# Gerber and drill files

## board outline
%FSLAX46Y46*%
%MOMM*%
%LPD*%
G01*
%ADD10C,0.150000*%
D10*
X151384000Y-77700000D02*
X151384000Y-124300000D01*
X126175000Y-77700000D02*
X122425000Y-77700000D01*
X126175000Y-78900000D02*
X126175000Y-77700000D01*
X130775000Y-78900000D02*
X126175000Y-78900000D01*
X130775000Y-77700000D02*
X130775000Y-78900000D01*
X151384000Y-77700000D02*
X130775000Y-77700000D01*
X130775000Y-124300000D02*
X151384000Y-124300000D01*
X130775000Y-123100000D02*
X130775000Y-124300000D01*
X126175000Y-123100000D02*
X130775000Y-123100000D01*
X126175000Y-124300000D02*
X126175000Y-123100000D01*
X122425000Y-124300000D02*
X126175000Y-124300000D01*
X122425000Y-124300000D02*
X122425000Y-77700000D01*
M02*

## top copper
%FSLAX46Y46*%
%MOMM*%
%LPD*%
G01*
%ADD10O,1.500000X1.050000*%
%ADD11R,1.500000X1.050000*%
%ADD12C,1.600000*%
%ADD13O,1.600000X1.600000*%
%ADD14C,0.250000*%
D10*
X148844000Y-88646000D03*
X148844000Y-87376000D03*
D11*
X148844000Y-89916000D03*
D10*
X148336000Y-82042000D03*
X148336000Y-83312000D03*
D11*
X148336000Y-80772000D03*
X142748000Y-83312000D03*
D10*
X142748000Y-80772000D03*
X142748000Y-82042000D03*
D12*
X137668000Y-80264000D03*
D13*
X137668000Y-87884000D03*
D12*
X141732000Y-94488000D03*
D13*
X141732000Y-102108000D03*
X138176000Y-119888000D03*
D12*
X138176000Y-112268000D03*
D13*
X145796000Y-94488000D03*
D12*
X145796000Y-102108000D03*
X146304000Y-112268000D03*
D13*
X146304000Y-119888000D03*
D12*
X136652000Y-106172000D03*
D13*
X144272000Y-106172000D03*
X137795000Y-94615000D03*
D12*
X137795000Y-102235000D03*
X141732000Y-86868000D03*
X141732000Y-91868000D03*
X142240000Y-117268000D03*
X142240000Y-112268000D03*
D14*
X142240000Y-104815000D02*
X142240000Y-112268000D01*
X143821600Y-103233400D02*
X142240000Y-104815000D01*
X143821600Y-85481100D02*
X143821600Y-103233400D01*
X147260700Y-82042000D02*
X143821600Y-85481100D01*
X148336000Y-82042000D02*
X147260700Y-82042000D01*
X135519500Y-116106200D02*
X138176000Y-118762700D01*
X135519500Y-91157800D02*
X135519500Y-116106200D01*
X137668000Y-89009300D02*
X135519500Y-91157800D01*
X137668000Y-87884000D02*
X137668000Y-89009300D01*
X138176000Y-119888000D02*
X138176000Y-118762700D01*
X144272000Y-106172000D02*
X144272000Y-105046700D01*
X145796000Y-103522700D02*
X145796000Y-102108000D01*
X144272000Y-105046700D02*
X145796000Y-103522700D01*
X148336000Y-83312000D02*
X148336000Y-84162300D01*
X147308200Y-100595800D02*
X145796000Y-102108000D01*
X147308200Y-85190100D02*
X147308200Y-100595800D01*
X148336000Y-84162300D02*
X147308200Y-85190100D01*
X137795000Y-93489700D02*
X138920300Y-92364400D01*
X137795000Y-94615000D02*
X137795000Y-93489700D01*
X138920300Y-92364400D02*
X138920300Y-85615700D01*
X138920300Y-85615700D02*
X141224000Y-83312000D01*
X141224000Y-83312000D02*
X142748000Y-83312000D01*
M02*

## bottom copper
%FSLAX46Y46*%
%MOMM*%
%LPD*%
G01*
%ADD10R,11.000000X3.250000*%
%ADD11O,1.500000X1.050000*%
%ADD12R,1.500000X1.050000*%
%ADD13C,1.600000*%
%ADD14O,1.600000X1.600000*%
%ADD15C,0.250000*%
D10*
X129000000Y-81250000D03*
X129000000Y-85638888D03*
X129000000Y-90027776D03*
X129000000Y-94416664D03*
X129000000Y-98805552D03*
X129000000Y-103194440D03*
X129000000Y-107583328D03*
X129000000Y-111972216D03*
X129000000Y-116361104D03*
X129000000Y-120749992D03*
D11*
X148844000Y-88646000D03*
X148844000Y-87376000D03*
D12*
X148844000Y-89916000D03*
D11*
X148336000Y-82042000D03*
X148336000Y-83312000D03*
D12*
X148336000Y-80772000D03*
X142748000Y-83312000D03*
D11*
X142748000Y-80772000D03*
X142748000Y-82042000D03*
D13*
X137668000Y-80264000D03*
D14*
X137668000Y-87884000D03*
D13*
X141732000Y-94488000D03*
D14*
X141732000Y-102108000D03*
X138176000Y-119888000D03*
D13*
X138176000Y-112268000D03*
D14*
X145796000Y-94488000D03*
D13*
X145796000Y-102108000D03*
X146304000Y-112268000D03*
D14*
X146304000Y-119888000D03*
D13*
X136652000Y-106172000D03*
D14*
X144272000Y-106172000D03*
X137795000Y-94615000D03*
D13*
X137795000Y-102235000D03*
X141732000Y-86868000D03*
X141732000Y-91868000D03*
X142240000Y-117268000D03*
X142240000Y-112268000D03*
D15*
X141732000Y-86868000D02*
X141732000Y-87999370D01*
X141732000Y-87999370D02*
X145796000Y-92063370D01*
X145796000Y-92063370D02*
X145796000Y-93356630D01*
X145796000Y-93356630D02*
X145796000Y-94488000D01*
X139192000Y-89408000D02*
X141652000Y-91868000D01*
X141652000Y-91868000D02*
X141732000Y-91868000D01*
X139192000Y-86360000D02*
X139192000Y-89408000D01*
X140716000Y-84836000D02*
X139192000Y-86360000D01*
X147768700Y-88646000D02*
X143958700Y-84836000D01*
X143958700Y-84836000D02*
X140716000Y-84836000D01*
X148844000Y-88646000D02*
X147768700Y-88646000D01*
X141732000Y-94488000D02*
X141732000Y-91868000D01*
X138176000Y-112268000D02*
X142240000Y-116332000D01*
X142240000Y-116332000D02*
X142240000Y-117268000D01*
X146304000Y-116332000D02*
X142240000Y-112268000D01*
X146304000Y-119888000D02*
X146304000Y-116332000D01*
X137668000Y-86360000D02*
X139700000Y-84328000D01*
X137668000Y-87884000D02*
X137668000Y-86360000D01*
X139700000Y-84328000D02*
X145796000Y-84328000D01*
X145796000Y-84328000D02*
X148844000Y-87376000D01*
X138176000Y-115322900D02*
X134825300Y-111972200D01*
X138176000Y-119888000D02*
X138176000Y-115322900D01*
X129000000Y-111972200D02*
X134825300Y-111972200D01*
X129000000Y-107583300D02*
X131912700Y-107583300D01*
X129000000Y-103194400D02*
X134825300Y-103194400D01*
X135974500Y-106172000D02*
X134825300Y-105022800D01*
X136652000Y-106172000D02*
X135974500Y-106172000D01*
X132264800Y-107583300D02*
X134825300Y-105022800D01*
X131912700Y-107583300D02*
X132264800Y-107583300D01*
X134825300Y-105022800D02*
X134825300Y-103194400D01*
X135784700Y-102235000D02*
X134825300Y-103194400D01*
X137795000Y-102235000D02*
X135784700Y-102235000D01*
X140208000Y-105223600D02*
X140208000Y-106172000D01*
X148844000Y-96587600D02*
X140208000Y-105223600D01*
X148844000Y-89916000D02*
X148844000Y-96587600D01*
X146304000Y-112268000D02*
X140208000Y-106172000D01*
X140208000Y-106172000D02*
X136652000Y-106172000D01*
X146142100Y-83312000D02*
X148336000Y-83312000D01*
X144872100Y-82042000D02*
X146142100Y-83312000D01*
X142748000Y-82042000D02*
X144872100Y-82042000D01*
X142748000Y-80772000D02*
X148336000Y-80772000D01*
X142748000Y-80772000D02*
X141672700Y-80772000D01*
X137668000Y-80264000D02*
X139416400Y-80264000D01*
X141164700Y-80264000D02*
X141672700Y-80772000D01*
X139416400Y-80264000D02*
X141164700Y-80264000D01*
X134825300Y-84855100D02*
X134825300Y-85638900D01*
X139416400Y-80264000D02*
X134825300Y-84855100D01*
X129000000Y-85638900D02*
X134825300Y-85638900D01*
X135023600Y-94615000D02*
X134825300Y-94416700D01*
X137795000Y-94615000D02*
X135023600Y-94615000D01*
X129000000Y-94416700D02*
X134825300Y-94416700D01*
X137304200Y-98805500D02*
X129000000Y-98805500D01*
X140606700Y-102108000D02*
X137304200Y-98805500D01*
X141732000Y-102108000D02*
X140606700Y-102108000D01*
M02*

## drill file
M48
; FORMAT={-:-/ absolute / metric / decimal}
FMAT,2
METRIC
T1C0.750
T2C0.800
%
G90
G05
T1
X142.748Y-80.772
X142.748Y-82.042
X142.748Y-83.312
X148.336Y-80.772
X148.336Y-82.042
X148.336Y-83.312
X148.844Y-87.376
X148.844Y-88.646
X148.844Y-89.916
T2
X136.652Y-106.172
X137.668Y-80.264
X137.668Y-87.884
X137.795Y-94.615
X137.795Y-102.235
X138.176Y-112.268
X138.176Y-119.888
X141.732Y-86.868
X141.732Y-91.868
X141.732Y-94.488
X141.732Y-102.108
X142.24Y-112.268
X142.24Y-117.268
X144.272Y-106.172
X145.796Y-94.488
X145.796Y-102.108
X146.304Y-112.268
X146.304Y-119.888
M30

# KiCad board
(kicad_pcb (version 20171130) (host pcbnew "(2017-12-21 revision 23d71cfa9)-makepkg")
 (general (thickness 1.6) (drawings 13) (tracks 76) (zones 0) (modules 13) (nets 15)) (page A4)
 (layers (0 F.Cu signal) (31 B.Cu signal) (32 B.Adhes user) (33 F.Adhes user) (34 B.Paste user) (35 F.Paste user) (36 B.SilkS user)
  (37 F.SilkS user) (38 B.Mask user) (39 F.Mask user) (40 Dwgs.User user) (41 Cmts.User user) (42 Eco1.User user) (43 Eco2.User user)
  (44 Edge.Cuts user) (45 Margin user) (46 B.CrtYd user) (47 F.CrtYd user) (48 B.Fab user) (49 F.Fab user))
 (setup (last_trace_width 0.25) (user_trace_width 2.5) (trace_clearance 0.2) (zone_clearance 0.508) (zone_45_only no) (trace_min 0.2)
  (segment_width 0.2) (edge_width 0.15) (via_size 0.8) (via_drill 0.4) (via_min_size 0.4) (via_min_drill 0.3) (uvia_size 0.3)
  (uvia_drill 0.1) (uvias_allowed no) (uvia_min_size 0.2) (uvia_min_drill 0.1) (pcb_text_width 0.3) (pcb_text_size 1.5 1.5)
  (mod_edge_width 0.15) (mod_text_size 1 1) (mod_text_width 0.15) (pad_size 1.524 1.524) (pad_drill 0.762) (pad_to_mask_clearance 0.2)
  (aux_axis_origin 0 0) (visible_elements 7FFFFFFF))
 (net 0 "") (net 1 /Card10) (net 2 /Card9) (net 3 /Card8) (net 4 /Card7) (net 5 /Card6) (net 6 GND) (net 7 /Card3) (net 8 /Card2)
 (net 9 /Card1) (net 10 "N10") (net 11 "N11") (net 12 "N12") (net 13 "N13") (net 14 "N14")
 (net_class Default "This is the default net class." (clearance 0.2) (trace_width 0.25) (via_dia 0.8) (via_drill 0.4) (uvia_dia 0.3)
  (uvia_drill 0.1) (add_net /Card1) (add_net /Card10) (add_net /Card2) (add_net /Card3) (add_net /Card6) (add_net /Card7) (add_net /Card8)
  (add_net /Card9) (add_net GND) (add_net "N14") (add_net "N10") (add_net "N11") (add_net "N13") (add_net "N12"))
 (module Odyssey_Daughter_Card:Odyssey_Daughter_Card (layer F.Cu) (at 129 101)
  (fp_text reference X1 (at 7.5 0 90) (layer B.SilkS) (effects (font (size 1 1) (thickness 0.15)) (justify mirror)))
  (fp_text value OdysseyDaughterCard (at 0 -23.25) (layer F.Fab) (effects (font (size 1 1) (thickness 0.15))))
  (pad 10 smd rect (at 0 -19.75) (size 11 3.25) (layers B.Cu B.Mask) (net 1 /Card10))
  (pad 9 smd rect (at 0 -15.361112) (size 11 3.25) (layers B.Cu B.Mask) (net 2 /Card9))
  (pad 8 smd rect (at 0 -10.972224) (size 11 3.25) (layers B.Cu B.Mask) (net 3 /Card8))
  (pad 7 smd rect (at 0 -6.583336) (size 11 3.25) (layers B.Cu B.Mask) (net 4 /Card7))
  (pad 6 smd rect (at 0 -2.194448) (size 11 3.25) (layers B.Cu B.Mask) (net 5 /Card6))
  (pad 5 smd rect (at 0 2.19444) (size 11 3.25) (layers B.Cu B.Mask) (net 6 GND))
  (pad 4 smd rect (at 0 6.583328) (size 11 3.25) (layers B.Cu B.Mask) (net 6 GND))
  (pad 3 smd rect (at 0 10.972216) (size 11 3.25) (layers B.Cu B.Mask) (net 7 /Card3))
  (pad 2 smd rect (at 0 15.361104) (size 11 3.25) (layers B.Cu B.Mask) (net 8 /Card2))
  (pad 1 smd rect (at 0 19.749992) (size 11 3.25) (layers B.Cu B.Mask) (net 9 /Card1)))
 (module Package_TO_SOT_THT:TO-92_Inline (layer F.Cu) (at 148.844 89.916 90)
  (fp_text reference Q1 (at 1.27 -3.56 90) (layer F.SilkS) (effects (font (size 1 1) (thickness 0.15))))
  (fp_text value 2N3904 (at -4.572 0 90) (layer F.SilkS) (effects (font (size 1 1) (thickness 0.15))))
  (pad 2 thru_hole oval (at 1.27 0 90) (size 1.05 1.5) (drill 0.75) (layers *.Cu *.Mask) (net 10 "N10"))
  (pad 3 thru_hole oval (at 2.54 0 90) (size 1.05 1.5) (drill 0.75) (layers *.Cu *.Mask) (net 7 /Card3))
  (pad 1 thru_hole rect (at 0 0 90) (size 1.05 1.5) (drill 0.75) (layers *.Cu *.Mask) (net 6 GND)))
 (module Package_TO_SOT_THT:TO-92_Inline (layer F.Cu) (at 148.336 80.772 270)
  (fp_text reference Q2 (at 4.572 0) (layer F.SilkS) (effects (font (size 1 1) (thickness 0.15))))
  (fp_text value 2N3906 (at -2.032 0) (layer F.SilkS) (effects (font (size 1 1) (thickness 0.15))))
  (pad 2 thru_hole oval (at 1.27 0 270) (size 1.05 1.5) (drill 0.75) (layers *.Cu *.Mask) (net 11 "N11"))
  (pad 3 thru_hole oval (at 2.54 0 270) (size 1.05 1.5) (drill 0.75) (layers *.Cu *.Mask) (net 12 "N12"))
  (pad 1 thru_hole rect (at 0 0 270) (size 1.05 1.5) (drill 0.75) (layers *.Cu *.Mask) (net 2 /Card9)))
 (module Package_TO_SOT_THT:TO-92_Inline (layer F.Cu) (at 142.748 83.312 90)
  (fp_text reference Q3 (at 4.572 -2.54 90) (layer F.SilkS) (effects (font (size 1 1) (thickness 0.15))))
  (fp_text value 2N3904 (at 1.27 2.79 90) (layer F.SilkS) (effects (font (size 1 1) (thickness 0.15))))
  (pad 1 thru_hole rect (at 0 0 90) (size 1.05 1.5) (drill 0.75) (layers *.Cu *.Mask) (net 4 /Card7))
  (pad 3 thru_hole oval (at 2.54 0 90) (size 1.05 1.5) (drill 0.75) (layers *.Cu *.Mask) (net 2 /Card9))
  (pad 2 thru_hole oval (at 1.27 0 90) (size 1.05 1.5) (drill 0.75) (layers *.Cu *.Mask) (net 12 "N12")))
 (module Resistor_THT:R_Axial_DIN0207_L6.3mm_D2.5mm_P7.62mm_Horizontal (layer F.Cu) (at 137.668 80.264 270)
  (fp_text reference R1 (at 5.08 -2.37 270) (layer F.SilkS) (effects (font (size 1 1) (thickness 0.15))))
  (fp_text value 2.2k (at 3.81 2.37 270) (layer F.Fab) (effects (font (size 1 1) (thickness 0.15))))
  (pad 1 thru_hole circle (at 0 0 270) (size 1.6 1.6) (drill 0.8) (layers *.Cu *.Mask) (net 2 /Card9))
  (pad 2 thru_hole oval (at 7.62 0 270) (size 1.6 1.6) (drill 0.8) (layers *.Cu *.Mask) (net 7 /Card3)))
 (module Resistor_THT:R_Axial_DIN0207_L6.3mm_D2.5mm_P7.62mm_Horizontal (layer F.Cu) (at 141.732 94.488 270)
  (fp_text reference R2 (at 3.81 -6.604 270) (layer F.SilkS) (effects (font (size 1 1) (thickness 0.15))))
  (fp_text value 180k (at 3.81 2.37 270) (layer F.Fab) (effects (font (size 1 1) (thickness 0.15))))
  (pad 1 thru_hole circle (at 0 0 270) (size 1.6 1.6) (drill 0.8) (layers *.Cu *.Mask) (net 10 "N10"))
  (pad 2 thru_hole oval (at 7.62 0 270) (size 1.6 1.6) (drill 0.8) (layers *.Cu *.Mask) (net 5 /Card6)))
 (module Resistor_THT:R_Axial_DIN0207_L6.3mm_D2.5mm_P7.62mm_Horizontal (layer F.Cu) (at 138.176 112.268 270)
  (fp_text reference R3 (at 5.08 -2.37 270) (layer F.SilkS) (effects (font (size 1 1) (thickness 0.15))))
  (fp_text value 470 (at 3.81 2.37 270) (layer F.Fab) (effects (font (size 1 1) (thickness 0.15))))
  (pad 2 thru_hole oval (at 7.62 0 270) (size 1.6 1.6) (drill 0.8) (layers *.Cu *.Mask) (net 7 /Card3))
  (pad 1 thru_hole circle (at 0 0 270) (size 1.6 1.6) (drill 0.8) (layers *.Cu *.Mask) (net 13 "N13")))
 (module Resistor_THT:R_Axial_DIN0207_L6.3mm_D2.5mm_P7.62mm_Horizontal (layer F.Cu) (at 145.796 102.108 90)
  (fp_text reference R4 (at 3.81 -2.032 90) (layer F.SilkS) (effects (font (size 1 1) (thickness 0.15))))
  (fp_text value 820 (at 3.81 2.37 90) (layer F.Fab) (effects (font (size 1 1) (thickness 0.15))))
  (pad 2 thru_hole oval (at 7.62 0 90) (size 1.6 1.6) (drill 0.8) (layers *.Cu *.Mask) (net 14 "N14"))
  (pad 1 thru_hole circle (at 0 0 90) (size 1.6 1.6) (drill 0.8) (layers *.Cu *.Mask) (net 12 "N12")))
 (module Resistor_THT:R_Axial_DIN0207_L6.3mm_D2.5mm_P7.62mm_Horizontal (layer F.Cu) (at 146.304 112.268 270)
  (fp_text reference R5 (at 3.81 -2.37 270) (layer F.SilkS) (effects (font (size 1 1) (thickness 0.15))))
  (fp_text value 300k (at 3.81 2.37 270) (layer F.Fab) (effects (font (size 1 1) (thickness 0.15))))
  (pad 1 thru_hole circle (at 0 0 270) (size 1.6 1.6) (drill 0.8) (layers *.Cu *.Mask) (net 6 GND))
  (pad 2 thru_hole oval (at 7.62 0 270) (size 1.6 1.6) (drill 0.8) (layers *.Cu *.Mask) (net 11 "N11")))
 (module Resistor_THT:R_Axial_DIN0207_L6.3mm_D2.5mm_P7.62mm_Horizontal (layer F.Cu) (at 136.652 106.172)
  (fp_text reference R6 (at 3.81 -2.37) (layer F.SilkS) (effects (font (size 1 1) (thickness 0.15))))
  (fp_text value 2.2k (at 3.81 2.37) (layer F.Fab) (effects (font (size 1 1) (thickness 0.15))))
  (pad 1 thru_hole circle (at 0 0) (size 1.6 1.6) (drill 0.8) (layers *.Cu *.Mask) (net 6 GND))
  (pad 2 thru_hole oval (at 7.62 0) (size 1.6 1.6) (drill 0.8) (layers *.Cu *.Mask) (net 12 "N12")))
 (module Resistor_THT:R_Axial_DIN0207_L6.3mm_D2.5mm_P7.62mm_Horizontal (layer F.Cu) (at 137.795 102.235 90)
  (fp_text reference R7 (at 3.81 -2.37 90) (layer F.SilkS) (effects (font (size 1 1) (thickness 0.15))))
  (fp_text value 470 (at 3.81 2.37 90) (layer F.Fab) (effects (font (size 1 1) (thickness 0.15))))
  (pad 2 thru_hole oval (at 7.62 0 90) (size 1.6 1.6) (drill 0.8) (layers *.Cu *.Mask) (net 4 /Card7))
  (pad 1 thru_hole circle (at 0 0 90) (size 1.6 1.6) (drill 0.8) (layers *.Cu *.Mask) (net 6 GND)))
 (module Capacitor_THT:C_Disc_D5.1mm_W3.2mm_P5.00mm (layer F.Cu) (at 141.732 86.868 270)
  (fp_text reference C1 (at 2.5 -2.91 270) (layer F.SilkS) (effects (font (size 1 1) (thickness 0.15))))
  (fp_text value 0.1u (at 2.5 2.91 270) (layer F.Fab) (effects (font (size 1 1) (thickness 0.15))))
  (pad 1 thru_hole circle (at 0 0 270) (size 1.6 1.6) (drill 0.8) (layers *.Cu *.Mask) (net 14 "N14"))
  (pad 2 thru_hole circle (at 5 0 270) (size 1.6 1.6) (drill 0.8) (layers *.Cu *.Mask) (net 10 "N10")))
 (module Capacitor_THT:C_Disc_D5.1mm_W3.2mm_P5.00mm (layer F.Cu) (at 142.24 112.268 270)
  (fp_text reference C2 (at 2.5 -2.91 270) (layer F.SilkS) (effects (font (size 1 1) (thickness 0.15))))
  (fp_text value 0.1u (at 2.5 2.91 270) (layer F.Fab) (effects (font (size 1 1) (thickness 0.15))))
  (pad 2 thru_hole circle (at 5 0 270) (size 1.6 1.6) (drill 0.8) (layers *.Cu *.Mask) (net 13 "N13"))
  (pad 1 thru_hole circle (at 0 0 270) (size 1.6 1.6) (drill 0.8) (layers *.Cu *.Mask) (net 11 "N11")))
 (gr_line (start 151.384 77.7) (end 151.384 124.3) (layer Edge.Cuts) (width 0.15))
 (gr_line (start 126.175 77.7) (end 122.425 77.7) (layer Edge.Cuts) (width 0.15))
 (gr_line (start 126.175 78.9) (end 126.175 77.7) (layer Edge.Cuts) (width 0.15))
 (gr_line (start 130.775 78.9) (end 126.175 78.9) (layer Edge.Cuts) (width 0.15))
 (gr_line (start 130.775 77.7) (end 130.775 78.9) (layer Edge.Cuts) (width 0.15))
 (gr_line (start 151.384 77.7) (end 130.775 77.7) (layer Edge.Cuts) (width 0.15))
 (gr_line (start 130.775 124.3) (end 151.384 124.3) (layer Edge.Cuts) (width 0.15))
 (gr_line (start 130.775 123.1) (end 130.775 124.3) (layer Edge.Cuts) (width 0.15))
 (gr_line (start 126.175 123.1) (end 130.775 123.1) (layer Edge.Cuts) (width 0.15))
 (gr_line (start 126.175 124.3) (end 126.175 123.1) (layer Edge.Cuts) (width 0.15))
 (gr_line (start 122.425 124.3) (end 126.175 124.3) (layer Edge.Cuts) (width 0.15))
 (gr_line (start 122.425 124.3) (end 122.425 77.7) (layer Edge.Cuts) (width 0.15))
 (segment (start 141.732 86.868) (end 141.732 87.99937) (width 0.25) (layer B.Cu) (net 14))
 (segment (start 141.732 87.99937) (end 145.796 92.06337) (width 0.25) (layer B.Cu) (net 14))
 (segment (start 145.796 92.06337) (end 145.796 93.35663) (width 0.25) (layer B.Cu) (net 14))
 (segment (start 145.796 93.35663) (end 145.796 94.488) (width 0.25) (layer B.Cu) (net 14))
 (segment (start 139.192 89.408) (end 141.652 91.868) (width 0.25) (layer B.Cu) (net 10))
 (segment (start 141.652 91.868) (end 141.732 91.868) (width 0.25) (layer B.Cu) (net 10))
 (segment (start 139.192 86.36) (end 139.192 89.408) (width 0.25) (layer B.Cu) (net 10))
 (segment (start 140.716 84.836) (end 139.192 86.36) (width 0.25) (layer B.Cu) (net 10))
 (segment (start 147.7687 88.646) (end 143.9587 84.836) (width 0.25) (layer B.Cu) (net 10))
 (segment (start 143.9587 84.836) (end 140.716 84.836) (width 0.25) (layer B.Cu) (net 10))
 (segment (start 148.844 88.646) (end 147.7687 88.646) (width 0.25) (layer B.Cu) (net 10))
 (segment (start 141.732 94.488) (end 141.732 91.868) (width 0.25) (layer B.Cu) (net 10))
 (segment (start 138.176 112.268) (end 142.24 116.332) (width 0.25) (layer B.Cu) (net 13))
 (segment (start 142.24 116.332) (end 142.24 117.268) (width 0.25) (layer B.Cu) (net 13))
 (segment (start 146.304 116.332) (end 142.24 112.268) (width 0.25) (layer B.Cu) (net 11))
 (segment (start 146.304 119.888) (end 146.304 116.332) (width 0.25) (layer B.Cu) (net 11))
 (segment (start 142.24 104.815) (end 142.24 112.268) (width 0.25) (layer F.Cu) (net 11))
 (segment (start 143.8216 103.2334) (end 142.24 104.815) (width 0.25) (layer F.Cu) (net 11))
 (segment (start 143.8216 85.4811) (end 143.8216 103.2334) (width 0.25) (layer F.Cu) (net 11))
 (segment (start 147.2607 82.042) (end 143.8216 85.4811) (width 0.25) (layer F.Cu) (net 11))
 (segment (start 148.336 82.042) (end 147.2607 82.042) (width 0.25) (layer F.Cu) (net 11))
 (segment (start 137.668 86.36) (end 139.7 84.328) (width 0.25) (layer B.Cu) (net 7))
 (segment (start 137.668 87.884) (end 137.668 86.36) (width 0.25) (layer B.Cu) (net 7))
 (segment (start 139.7 84.328) (end 145.796 84.328) (width 0.25) (layer B.Cu) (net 7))
 (segment (start 145.796 84.328) (end 148.844 87.376) (width 0.25) (layer B.Cu) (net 7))
 (segment (start 135.5195 116.1062) (end 138.176 118.7627) (width 0.25) (layer F.Cu) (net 7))
 (segment (start 135.5195 91.1578) (end 135.5195 116.1062) (width 0.25) (layer F.Cu) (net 7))
 (segment (start 137.668 89.0093) (end 135.5195 91.1578) (width 0.25) (layer F.Cu) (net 7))
 (segment (start 137.668 87.884) (end 137.668 89.0093) (width 0.25) (layer F.Cu) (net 7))
 (segment (start 138.176 119.888) (end 138.176 118.7627) (width 0.25) (layer F.Cu) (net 7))
 (segment (start 138.176 115.3229) (end 134.8253 111.9722) (width 0.25) (layer B.Cu) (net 7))
 (segment (start 138.176 119.888) (end 138.176 115.3229) (width 0.25) (layer B.Cu) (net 7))
 (segment (start 129 111.9722) (end 134.8253 111.9722) (width 0.25) (layer B.Cu) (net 7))
 (segment (start 129 107.5833) (end 131.9127 107.5833) (width 0.25) (layer B.Cu) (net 6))
 (segment (start 129 103.1944) (end 134.8253 103.1944) (width 0.25) (layer B.Cu) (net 6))
 (segment (start 135.9745 106.172) (end 134.8253 105.0228) (width 0.25) (layer B.Cu) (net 6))
 (segment (start 136.652 106.172) (end 135.9745 106.172) (width 0.25) (layer B.Cu) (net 6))
 (segment (start 132.2648 107.5833) (end 134.8253 105.0228) (width 0.25) (layer B.Cu) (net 6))
 (segment (start 131.9127 107.5833) (end 132.2648 107.5833) (width 0.25) (layer B.Cu) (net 6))
 (segment (start 134.8253 105.0228) (end 134.8253 103.1944) (width 0.25) (layer B.Cu) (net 6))
 (segment (start 135.7847 102.235) (end 134.8253 103.1944) (width 0.25) (layer B.Cu) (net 6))
 (segment (start 137.795 102.235) (end 135.7847 102.235) (width 0.25) (layer B.Cu) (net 6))
 (segment (start 140.208 105.2236) (end 140.208 106.172) (width 0.25) (layer B.Cu) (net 6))
 (segment (start 148.844 96.5876) (end 140.208 105.2236) (width 0.25) (layer B.Cu) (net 6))
 (segment (start 148.844 89.916) (end 148.844 96.5876) (width 0.25) (layer B.Cu) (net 6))
 (segment (start 146.304 112.268) (end 140.208 106.172) (width 0.25) (layer B.Cu) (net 6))
 (segment (start 140.208 106.172) (end 136.652 106.172) (width 0.25) (layer B.Cu) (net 6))
 (segment (start 144.272 106.172) (end 144.272 105.0467) (width 0.25) (layer F.Cu) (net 12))
 (segment (start 145.796 103.5227) (end 145.796 102.108) (width 0.25) (layer F.Cu) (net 12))
 (segment (start 144.272 105.0467) (end 145.796 103.5227) (width 0.25) (layer F.Cu) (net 12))
 (segment (start 148.336 83.312) (end 148.336 84.1623) (width 0.25) (layer F.Cu) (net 12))
 (segment (start 146.1421 83.312) (end 148.336 83.312) (width 0.25) (layer B.Cu) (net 12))
 (segment (start 144.8721 82.042) (end 146.1421 83.312) (width 0.25) (layer B.Cu) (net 12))
 (segment (start 142.748 82.042) (end 144.8721 82.042) (width 0.25) (layer B.Cu) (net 12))
 (segment (start 147.3082 100.5958) (end 145.796 102.108) (width 0.25) (layer F.Cu) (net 12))
 (segment (start 147.3082 85.1901) (end 147.3082 100.5958) (width 0.25) (layer F.Cu) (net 12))
 (segment (start 148.336 84.1623) (end 147.3082 85.1901) (width 0.25) (layer F.Cu) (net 12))
 (segment (start 142.748 80.772) (end 148.336 80.772) (width 0.25) (layer B.Cu) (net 2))
 (segment (start 142.748 80.772) (end 141.6727 80.772) (width 0.25) (layer B.Cu) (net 2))
 (segment (start 137.668 80.264) (end 139.4164 80.264) (width 0.25) (layer B.Cu) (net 2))
 (segment (start 141.1647 80.264) (end 141.6727 80.772) (width 0.25) (layer B.Cu) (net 2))
 (segment (start 139.4164 80.264) (end 141.1647 80.264) (width 0.25) (layer B.Cu) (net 2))
 (segment (start 134.8253 84.8551) (end 134.8253 85.6389) (width 0.25) (layer B.Cu) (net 2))
 (segment (start 139.4164 80.264) (end 134.8253 84.8551) (width 0.25) (layer B.Cu) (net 2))
 (segment (start 129 85.6389) (end 134.8253 85.6389) (width 0.25) (layer B.Cu) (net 2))
 (segment (start 137.795 93.4897) (end 138.9203 92.3644) (width 0.25) (layer F.Cu) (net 4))
 (segment (start 137.795 94.615) (end 137.795 93.4897) (width 0.25) (layer F.Cu) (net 4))
 (segment (start 138.9203 92.3644) (end 138.9203 85.6157) (width 0.25) (layer F.Cu) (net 4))
 (segment (start 138.9203 85.6157) (end 141.224 83.312) (width 0.25) (layer F.Cu) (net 4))
 (segment (start 141.224 83.312) (end 142.748 83.312) (width 0.25) (layer F.Cu) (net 4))
 (segment (start 135.0236 94.615) (end 134.8253 94.4167) (width 0.25) (layer B.Cu) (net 4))
 (segment (start 137.795 94.615) (end 135.0236 94.615) (width 0.25) (layer B.Cu) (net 4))
 (segment (start 129 94.4167) (end 134.8253 94.4167) (width 0.25) (layer B.Cu) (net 4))
 (segment (start 137.3042 98.8055) (end 129 98.8055) (width 0.25) (layer B.Cu) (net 5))
 (segment (start 140.6067 102.108) (end 137.3042 98.8055) (width 0.25) (layer B.Cu) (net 5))
 (segment (start 141.732 102.108) (end 140.6067 102.108) (width 0.25) (layer B.Cu) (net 5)))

